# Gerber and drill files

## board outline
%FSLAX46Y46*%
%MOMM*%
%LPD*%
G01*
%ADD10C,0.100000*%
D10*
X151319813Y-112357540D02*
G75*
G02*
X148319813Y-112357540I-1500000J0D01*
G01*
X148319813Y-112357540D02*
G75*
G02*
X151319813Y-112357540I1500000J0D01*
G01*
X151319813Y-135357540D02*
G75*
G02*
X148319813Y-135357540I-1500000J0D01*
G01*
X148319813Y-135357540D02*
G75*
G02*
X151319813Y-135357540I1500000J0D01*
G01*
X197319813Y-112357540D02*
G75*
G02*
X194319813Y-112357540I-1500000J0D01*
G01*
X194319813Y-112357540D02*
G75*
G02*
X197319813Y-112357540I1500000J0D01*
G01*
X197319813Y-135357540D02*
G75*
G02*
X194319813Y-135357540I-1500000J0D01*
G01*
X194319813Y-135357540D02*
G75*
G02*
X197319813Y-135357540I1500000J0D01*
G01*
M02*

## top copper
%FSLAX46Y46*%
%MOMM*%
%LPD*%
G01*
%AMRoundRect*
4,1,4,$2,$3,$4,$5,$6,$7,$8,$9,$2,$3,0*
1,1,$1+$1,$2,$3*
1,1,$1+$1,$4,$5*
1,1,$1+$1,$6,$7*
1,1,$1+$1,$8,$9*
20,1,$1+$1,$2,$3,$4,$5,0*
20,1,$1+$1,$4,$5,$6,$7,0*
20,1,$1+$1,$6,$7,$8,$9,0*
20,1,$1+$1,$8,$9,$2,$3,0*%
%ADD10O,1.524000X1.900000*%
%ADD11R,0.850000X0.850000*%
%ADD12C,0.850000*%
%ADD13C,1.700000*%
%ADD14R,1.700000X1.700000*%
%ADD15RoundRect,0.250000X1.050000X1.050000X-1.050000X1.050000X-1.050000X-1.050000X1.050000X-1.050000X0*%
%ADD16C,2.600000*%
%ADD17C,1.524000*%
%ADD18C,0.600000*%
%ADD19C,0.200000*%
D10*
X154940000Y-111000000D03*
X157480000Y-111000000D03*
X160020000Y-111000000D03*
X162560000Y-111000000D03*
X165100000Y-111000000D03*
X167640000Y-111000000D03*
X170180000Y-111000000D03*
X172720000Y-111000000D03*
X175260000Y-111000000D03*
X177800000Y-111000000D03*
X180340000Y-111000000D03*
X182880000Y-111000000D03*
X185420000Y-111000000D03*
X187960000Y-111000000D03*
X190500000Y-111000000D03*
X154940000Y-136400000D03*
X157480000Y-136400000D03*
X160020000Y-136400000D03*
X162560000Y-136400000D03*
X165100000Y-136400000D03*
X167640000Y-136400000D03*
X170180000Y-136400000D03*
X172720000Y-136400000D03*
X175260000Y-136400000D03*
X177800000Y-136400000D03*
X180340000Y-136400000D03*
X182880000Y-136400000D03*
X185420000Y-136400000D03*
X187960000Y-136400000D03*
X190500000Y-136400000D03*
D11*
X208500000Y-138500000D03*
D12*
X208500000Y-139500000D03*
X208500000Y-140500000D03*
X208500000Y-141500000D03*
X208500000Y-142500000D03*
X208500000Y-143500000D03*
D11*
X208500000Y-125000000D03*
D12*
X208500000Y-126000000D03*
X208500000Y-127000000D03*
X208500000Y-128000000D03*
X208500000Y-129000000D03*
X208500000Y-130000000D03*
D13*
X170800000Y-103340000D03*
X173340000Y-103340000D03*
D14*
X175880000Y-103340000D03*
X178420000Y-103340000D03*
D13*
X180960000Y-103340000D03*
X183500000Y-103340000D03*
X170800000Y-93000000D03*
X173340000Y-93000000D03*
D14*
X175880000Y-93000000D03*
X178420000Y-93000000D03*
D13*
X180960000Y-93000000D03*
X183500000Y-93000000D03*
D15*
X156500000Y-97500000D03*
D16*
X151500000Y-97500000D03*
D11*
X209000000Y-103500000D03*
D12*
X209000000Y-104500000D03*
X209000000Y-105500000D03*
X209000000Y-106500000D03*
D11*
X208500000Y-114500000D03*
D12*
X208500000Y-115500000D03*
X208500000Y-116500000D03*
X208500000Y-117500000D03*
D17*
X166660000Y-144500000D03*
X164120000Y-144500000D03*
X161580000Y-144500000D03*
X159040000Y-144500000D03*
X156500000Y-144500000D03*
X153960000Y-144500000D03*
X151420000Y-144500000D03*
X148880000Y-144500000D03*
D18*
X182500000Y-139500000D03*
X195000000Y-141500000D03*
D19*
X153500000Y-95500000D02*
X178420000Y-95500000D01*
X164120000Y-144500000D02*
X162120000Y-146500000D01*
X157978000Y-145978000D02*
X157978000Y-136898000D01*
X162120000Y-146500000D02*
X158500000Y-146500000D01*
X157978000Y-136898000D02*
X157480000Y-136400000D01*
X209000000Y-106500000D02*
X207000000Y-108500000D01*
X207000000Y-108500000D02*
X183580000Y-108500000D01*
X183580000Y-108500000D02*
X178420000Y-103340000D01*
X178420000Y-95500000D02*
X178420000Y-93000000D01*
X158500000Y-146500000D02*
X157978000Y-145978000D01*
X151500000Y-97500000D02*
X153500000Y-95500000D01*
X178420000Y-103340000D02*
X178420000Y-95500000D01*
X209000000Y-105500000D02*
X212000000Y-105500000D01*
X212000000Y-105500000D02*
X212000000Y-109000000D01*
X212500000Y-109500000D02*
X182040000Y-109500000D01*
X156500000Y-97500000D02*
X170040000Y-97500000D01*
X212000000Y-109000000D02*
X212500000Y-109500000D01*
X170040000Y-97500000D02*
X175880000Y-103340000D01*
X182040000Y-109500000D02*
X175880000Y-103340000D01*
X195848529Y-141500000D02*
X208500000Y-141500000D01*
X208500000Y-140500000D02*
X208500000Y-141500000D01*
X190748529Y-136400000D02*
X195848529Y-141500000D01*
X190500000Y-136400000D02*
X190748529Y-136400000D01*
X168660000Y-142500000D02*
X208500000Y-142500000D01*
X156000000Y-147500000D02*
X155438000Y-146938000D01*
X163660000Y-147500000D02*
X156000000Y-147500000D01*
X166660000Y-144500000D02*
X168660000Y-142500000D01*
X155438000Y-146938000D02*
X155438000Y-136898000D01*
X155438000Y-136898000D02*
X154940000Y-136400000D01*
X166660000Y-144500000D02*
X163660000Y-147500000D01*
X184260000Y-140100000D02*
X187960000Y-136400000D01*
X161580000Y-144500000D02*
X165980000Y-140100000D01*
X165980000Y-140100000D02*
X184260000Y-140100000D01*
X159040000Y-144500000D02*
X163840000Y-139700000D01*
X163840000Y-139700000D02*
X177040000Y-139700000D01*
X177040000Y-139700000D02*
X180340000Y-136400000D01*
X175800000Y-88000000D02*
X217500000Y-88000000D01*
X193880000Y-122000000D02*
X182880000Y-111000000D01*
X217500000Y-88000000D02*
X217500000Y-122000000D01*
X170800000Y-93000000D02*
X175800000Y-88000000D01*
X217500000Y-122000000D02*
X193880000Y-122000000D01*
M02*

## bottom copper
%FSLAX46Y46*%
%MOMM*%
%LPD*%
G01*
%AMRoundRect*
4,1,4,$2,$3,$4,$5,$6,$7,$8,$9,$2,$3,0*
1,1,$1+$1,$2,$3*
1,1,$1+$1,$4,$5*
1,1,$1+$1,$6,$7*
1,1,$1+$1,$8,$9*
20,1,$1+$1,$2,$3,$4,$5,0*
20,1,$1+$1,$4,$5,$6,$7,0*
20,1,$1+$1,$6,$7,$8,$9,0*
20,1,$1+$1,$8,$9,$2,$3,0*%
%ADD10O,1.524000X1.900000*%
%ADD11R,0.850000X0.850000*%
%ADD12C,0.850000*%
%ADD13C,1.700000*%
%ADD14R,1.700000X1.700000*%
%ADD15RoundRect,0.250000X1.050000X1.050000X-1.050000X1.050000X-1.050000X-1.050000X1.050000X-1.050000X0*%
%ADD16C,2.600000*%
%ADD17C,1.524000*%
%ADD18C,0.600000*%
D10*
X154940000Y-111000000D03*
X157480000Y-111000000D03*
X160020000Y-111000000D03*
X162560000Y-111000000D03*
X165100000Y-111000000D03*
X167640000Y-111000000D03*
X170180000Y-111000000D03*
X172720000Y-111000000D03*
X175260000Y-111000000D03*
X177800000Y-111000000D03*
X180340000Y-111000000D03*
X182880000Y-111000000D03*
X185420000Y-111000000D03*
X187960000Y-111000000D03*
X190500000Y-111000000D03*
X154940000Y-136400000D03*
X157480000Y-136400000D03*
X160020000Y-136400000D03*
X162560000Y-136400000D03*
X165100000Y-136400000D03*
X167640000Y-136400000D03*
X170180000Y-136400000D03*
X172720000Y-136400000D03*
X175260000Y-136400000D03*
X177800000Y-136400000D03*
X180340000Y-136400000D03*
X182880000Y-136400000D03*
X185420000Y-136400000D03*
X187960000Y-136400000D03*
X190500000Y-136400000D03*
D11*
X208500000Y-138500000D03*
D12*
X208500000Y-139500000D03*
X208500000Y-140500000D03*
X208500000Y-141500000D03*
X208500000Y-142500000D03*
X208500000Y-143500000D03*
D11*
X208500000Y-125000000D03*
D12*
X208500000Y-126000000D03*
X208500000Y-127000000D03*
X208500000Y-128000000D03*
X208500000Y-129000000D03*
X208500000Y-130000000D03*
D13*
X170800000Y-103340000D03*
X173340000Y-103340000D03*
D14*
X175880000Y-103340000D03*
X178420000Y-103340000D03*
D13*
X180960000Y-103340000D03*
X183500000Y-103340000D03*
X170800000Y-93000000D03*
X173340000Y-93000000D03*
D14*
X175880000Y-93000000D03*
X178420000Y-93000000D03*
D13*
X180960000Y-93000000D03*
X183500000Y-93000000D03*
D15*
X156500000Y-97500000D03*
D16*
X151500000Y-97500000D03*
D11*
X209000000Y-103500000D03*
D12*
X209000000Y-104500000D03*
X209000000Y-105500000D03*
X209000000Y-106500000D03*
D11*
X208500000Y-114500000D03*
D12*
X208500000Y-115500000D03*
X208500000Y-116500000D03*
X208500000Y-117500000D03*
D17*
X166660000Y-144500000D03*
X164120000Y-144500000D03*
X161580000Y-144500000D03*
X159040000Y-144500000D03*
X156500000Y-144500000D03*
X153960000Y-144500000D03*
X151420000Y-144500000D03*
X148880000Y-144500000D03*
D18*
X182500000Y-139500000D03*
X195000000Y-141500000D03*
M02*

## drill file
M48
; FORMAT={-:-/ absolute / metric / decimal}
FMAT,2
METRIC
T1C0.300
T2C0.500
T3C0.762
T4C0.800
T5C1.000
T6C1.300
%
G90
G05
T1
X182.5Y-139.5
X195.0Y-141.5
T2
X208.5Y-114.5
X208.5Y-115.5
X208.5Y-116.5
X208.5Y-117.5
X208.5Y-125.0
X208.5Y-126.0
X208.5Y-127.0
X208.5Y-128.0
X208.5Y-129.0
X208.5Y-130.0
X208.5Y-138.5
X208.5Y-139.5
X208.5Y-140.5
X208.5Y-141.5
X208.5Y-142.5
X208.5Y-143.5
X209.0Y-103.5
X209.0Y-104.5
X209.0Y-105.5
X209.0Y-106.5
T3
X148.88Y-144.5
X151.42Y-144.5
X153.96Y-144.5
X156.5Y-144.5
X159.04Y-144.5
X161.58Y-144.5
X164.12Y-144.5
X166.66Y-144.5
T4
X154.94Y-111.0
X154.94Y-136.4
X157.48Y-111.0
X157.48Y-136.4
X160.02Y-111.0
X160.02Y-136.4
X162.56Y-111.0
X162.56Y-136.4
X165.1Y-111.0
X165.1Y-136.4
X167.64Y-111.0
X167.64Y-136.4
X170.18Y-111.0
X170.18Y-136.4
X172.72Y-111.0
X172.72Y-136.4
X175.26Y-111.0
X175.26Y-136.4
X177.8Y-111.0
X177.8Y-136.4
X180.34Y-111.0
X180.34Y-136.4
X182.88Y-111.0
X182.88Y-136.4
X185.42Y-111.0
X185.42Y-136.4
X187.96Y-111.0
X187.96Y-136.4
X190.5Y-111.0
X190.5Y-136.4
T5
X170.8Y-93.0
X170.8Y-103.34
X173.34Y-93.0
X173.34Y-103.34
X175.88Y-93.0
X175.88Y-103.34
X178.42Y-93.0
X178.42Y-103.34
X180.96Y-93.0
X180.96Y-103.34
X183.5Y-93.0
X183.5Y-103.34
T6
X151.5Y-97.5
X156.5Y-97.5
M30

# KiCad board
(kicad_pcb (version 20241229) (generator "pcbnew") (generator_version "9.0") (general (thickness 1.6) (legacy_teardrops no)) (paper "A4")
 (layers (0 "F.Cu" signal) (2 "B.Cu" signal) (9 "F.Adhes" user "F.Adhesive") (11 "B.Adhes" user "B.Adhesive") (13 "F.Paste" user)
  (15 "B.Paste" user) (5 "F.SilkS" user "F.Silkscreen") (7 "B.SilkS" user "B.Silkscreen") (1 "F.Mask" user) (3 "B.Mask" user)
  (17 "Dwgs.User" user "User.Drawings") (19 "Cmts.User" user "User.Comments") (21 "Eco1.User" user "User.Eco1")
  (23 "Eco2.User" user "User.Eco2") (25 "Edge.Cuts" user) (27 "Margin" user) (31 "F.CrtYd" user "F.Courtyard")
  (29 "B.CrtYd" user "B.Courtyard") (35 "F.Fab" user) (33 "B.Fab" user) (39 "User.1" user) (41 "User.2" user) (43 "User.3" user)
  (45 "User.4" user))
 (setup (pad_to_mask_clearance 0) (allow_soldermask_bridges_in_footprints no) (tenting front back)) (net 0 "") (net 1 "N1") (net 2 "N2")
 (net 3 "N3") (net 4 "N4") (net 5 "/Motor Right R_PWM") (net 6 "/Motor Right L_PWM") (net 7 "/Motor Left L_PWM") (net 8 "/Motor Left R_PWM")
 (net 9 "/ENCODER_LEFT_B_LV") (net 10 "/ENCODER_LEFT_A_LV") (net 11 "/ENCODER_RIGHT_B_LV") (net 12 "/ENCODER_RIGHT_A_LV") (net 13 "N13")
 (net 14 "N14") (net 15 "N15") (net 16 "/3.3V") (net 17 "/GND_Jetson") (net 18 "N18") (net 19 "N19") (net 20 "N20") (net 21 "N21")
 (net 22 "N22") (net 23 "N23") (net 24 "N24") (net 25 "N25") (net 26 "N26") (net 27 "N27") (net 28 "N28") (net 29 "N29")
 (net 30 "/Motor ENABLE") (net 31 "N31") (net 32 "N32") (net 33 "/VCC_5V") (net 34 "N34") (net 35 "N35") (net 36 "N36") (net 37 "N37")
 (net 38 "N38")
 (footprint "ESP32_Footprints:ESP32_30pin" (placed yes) (layer "F.Cu") (at 171.959813 122.92754 -90)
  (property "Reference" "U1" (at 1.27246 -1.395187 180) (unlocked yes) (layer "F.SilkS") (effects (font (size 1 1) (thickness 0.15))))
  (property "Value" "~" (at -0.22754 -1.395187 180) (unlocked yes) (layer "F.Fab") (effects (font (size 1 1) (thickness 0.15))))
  (fp_circle (center -10.57 22.14) (end -10.57 23.64) (stroke (width 0.1) (type default)) (fill no) (layer "Edge.Cuts"))
  (fp_circle (center 12.43 22.14) (end 12.43 23.64) (stroke (width 0.1) (type default)) (fill no) (layer "Edge.Cuts"))
  (fp_circle (center -10.57 -23.86) (end -10.57 -22.36) (stroke (width 0.1) (type default)) (fill no) (layer "Edge.Cuts"))
  (fp_circle (center 12.43 -23.86) (end 12.43 -22.36) (stroke (width 0.1) (type default)) (fill no) (layer "Edge.Cuts"))
  (pad "1" thru_hole oval (at -11.92754 17.019813 180) (size 1.524 1.9) (drill 0.8) (layers "*.Cu" "*.Mask") (remove_unused_layers no)
   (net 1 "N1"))
  (pad "2" thru_hole oval (at -11.92754 14.479813 180) (size 1.524 1.9) (drill 0.8) (layers "*.Cu" "*.Mask") (remove_unused_layers no)
   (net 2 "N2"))
  (pad "3" thru_hole oval (at -11.92754 11.939813 180) (size 1.524 1.9) (drill 0.8) (layers "*.Cu" "*.Mask") (remove_unused_layers no)
   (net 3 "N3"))
  (pad "4" thru_hole oval (at -11.92754 9.399813 180) (size 1.524 1.9) (drill 0.8) (layers "*.Cu" "*.Mask") (remove_unused_layers no)
   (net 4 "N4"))
  (pad "5" thru_hole oval (at -11.92754 6.859813 180) (size 1.524 1.9) (drill 0.8) (layers "*.Cu" "*.Mask") (remove_unused_layers no)
   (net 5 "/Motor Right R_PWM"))
  (pad "6" thru_hole oval (at -11.92754 4.319813 180) (size 1.524 1.9) (drill 0.8) (layers "*.Cu" "*.Mask") (remove_unused_layers no)
   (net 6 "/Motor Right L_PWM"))
  (pad "7" thru_hole oval (at -11.92754 1.779813 180) (size 1.524 1.9) (drill 0.8) (layers "*.Cu" "*.Mask") (remove_unused_layers no)
   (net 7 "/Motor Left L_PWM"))
  (pad "8" thru_hole oval (at -11.92754 -0.760187 180) (size 1.524 1.9) (drill 0.8) (layers "*.Cu" "*.Mask") (remove_unused_layers no)
   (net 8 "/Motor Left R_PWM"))
  (pad "9" thru_hole oval (at -11.92754 -3.300187 180) (size 1.524 1.9) (drill 0.8) (layers "*.Cu" "*.Mask") (remove_unused_layers no)
   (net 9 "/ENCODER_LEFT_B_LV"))
  (pad "10" thru_hole oval (at -11.92754 -5.840187 180) (size 1.524 1.9) (drill 0.8) (layers "*.Cu" "*.Mask") (remove_unused_layers no)
   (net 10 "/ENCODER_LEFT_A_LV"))
  (pad "11" thru_hole oval (at -11.92754 -8.380187 180) (size 1.524 1.9) (drill 0.8) (layers "*.Cu" "*.Mask") (remove_unused_layers no)
   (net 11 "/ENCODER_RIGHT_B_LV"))
  (pad "12" thru_hole oval (at -11.92754 -10.920187 180) (size 1.524 1.9) (drill 0.8) (layers "*.Cu" "*.Mask") (remove_unused_layers no)
   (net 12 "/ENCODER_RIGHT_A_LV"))
  (pad "13" thru_hole oval (at -11.92754 -13.460187 180) (size 1.524 1.9) (drill 0.8) (layers "*.Cu" "*.Mask") (remove_unused_layers no)
   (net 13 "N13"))
  (pad "14" thru_hole oval (at -11.92754 -16.000187 180) (size 1.524 1.9) (drill 0.8) (layers "*.Cu" "*.Mask") (remove_unused_layers no)
   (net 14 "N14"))
  (pad "15" thru_hole oval (at -11.92754 -18.540187 180) (size 1.524 1.9) (drill 0.8) (layers "*.Cu" "*.Mask") (remove_unused_layers no)
   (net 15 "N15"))
  (pad "16" thru_hole oval (at 13.47246 17.019813 180) (size 1.524 1.9) (drill 0.8) (layers "*.Cu" "*.Mask") (remove_unused_layers no)
   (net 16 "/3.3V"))
  (pad "17" thru_hole oval (at 13.47246 14.479813 180) (size 1.524 1.9) (drill 0.8) (layers "*.Cu" "*.Mask") (remove_unused_layers no)
   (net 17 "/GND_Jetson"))
  (pad "18" thru_hole oval (at 13.47246 11.939813 180) (size 1.524 1.9) (drill 0.8) (layers "*.Cu" "*.Mask") (remove_unused_layers no)
   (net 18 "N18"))
  (pad "19" thru_hole oval (at 13.47246 9.399813 180) (size 1.524 1.9) (drill 0.8) (layers "*.Cu" "*.Mask") (remove_unused_layers no)
   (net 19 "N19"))
  (pad "20" thru_hole oval (at 13.47246 6.859813 180) (size 1.524 1.9) (drill 0.8) (layers "*.Cu" "*.Mask" "Dwgs.User")
   (remove_unused_layers no) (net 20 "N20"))
  (pad "21" thru_hole oval (at 13.47246 4.319813 180) (size 1.524 1.9) (drill 0.8) (layers "*.Cu" "*.Mask") (remove_unused_layers no)
   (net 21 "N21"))
  (pad "22" thru_hole oval (at 13.47246 1.779813 180) (size 1.524 1.9) (drill 0.8) (layers "*.Cu" "*.Mask") (remove_unused_layers no)
   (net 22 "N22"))
  (pad "23" thru_hole oval (at 13.47246 -0.760187 180) (size 1.524 1.9) (drill 0.8) (layers "*.Cu" "*.Mask") (remove_unused_layers no)
   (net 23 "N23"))
  (pad "24" thru_hole oval (at 13.47246 -3.300187 180) (size 1.524 1.9) (drill 0.8) (layers "*.Cu" "*.Mask") (remove_unused_layers no)
   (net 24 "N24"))
  (pad "25" thru_hole oval (at 13.47246 -5.840187 180) (size 1.524 1.9) (drill 0.8) (layers "*.Cu" "*.Mask") (remove_unused_layers no)
   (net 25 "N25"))
  (pad "26" thru_hole oval (at 13.47246 -8.380187 180) (size 1.524 1.9) (drill 0.8) (layers "*.Cu" "*.Mask") (remove_unused_layers no)
   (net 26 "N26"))
  (pad "27" thru_hole oval (at 13.47246 -10.920187 180) (size 1.524 1.9) (drill 0.8) (layers "*.Cu" "*.Mask") (remove_unused_layers no)
   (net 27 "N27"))
  (pad "28" thru_hole oval (at 13.47246 -13.460187 180) (size 1.524 1.9) (drill 0.8) (layers "*.Cu" "*.Mask") (remove_unused_layers no)
   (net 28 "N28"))
  (pad "29" thru_hole oval (at 13.47246 -16.000187 180) (size 1.524 1.9) (drill 0.8) (layers "*.Cu" "*.Mask") (remove_unused_layers no)
   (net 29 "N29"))
  (pad "30" thru_hole oval (at 13.47246 -18.540187 180) (size 1.524 1.9) (drill 0.8) (layers "*.Cu" "*.Mask") (remove_unused_layers no)
   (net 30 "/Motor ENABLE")))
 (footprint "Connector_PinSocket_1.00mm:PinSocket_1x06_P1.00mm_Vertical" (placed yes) (layer "F.Cu") (at 208.5 138.5)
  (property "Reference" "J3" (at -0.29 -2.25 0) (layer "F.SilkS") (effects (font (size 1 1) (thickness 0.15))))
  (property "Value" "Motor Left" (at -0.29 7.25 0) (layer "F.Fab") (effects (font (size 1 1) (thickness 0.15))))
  (pad "1" thru_hole rect (at 0 0) (size 0.85 0.85) (drill 0.5) (layers "*.Cu" "*.Mask") (remove_unused_layers no)
   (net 8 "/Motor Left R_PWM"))
  (pad "2" thru_hole circle (at 0 1) (size 0.85 0.85) (drill 0.5) (layers "*.Cu" "*.Mask") (remove_unused_layers no)
   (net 7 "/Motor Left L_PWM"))
  (pad "3" thru_hole circle (at 0 2) (size 0.85 0.85) (drill 0.5) (layers "*.Cu" "*.Mask") (remove_unused_layers no)
   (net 30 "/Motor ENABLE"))
  (pad "4" thru_hole circle (at 0 3) (size 0.85 0.85) (drill 0.5) (layers "*.Cu" "*.Mask") (remove_unused_layers no)
   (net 30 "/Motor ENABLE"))
  (pad "5" thru_hole circle (at 0 4) (size 0.85 0.85) (drill 0.5) (layers "*.Cu" "*.Mask") (remove_unused_layers no) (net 16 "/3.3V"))
  (pad "6" thru_hole circle (at 0 5) (size 0.85 0.85) (drill 0.5) (layers "*.Cu" "*.Mask") (remove_unused_layers no) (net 17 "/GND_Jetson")))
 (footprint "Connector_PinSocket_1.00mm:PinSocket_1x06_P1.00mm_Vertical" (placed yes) (layer "F.Cu") (at 208.5 125)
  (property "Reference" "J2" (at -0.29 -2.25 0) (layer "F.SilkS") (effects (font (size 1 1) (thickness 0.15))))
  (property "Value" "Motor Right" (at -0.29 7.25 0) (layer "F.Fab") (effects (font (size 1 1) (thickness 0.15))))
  (pad "1" thru_hole rect (at 0 0) (size 0.85 0.85) (drill 0.5) (layers "*.Cu" "*.Mask") (remove_unused_layers no)
   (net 5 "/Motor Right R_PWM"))
  (pad "2" thru_hole circle (at 0 1) (size 0.85 0.85) (drill 0.5) (layers "*.Cu" "*.Mask") (remove_unused_layers no)
   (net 6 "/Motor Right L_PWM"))
  (pad "3" thru_hole circle (at 0 2) (size 0.85 0.85) (drill 0.5) (layers "*.Cu" "*.Mask") (remove_unused_layers no)
   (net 30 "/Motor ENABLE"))
  (pad "4" thru_hole circle (at 0 3) (size 0.85 0.85) (drill 0.5) (layers "*.Cu" "*.Mask") (remove_unused_layers no)
   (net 30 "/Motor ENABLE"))
  (pad "5" thru_hole circle (at 0 4) (size 0.85 0.85) (drill 0.5) (layers "*.Cu" "*.Mask") (remove_unused_layers no) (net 16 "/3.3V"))
  (pad "6" thru_hole circle (at 0 5) (size 0.85 0.85) (drill 0.5) (layers "*.Cu" "*.Mask") (remove_unused_layers no) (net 17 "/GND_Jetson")))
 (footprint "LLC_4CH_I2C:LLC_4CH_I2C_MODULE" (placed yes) (layer "F.Cu") (at 177.15 98.17 90)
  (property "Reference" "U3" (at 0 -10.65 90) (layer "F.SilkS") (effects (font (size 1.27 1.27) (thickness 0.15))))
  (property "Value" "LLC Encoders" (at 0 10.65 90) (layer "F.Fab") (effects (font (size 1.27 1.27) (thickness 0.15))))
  (pad "1" thru_hole circle (at -5.17 -6.35 90) (size 1.7 1.7) (drill 1) (layers "*.Cu" "*.Mask") (remove_unused_layers no) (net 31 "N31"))
  (pad "2" thru_hole circle (at -5.17 -3.81 90) (size 1.7 1.7) (drill 1) (layers "*.Cu" "*.Mask") (remove_unused_layers no) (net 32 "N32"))
  (pad "3" thru_hole rect (at -5.17 -1.27 90) (size 1.7 1.7) (drill 1) (layers "*.Cu" "*.Mask") (remove_unused_layers no) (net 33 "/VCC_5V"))
  (pad "4" thru_hole rect (at -5.17 1.27 90) (size 1.7 1.7) (drill 1) (layers "*.Cu" "*.Mask") (remove_unused_layers no)
   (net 17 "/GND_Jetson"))
  (pad "5" thru_hole circle (at -5.17 3.81 90) (size 1.7 1.7) (drill 1) (layers "*.Cu" "*.Mask") (remove_unused_layers no) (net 32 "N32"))
  (pad "6" thru_hole circle (at -5.17 6.35 90) (size 1.7 1.7) (drill 1) (layers "*.Cu" "*.Mask") (remove_unused_layers no) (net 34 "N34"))
  (pad "7" thru_hole circle (at 5.17 -6.35 90) (size 1.7 1.7) (drill 1) (layers "*.Cu" "*.Mask") (remove_unused_layers no)
   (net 12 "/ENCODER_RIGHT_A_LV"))
  (pad "8" thru_hole circle (at 5.17 -3.81 90) (size 1.7 1.7) (drill 1) (layers "*.Cu" "*.Mask") (remove_unused_layers no)
   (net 11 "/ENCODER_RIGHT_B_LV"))
  (pad "9" thru_hole rect (at 5.17 -1.27 90) (size 1.7 1.7) (drill 1) (layers "*.Cu" "*.Mask") (remove_unused_layers no) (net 16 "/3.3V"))
  (pad "10" thru_hole rect (at 5.17 1.27 90) (size 1.7 1.7) (drill 1) (layers "*.Cu" "*.Mask") (remove_unused_layers no)
   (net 17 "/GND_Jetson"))
  (pad "11" thru_hole circle (at 5.17 3.81 90) (size 1.7 1.7) (drill 1) (layers "*.Cu" "*.Mask") (remove_unused_layers no)
   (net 10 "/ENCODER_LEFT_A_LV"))
  (pad "12" thru_hole circle (at 5.17 6.35 90) (size 1.7 1.7) (drill 1) (layers "*.Cu" "*.Mask") (remove_unused_layers no)
   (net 9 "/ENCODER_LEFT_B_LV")))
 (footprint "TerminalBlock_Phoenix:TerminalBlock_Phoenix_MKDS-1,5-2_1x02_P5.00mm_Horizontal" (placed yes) (layer "F.Cu") (at 156.5 97.5 180)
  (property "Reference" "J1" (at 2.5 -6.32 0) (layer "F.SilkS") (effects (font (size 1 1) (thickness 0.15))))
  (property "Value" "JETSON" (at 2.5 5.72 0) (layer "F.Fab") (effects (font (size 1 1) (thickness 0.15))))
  (pad "1" thru_hole roundrect (at 0 0 180) (size 2.6 2.6) (drill 1.3) (layers "*.Cu" "*.Mask") (remove_unused_layers no)
   (roundrect_rratio 0.096154) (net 33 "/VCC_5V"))
  (pad "2" thru_hole circle (at 5 0 180) (size 2.6 2.6) (drill 1.3) (layers "*.Cu" "*.Mask") (remove_unused_layers no)
   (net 17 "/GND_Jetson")))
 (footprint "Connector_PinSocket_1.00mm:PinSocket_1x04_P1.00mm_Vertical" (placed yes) (layer "F.Cu") (at 209 103.5)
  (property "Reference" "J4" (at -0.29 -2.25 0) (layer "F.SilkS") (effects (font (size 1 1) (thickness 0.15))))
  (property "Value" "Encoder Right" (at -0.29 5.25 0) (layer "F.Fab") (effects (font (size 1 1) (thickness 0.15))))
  (pad "1" thru_hole rect (at 0 0) (size 0.85 0.85) (drill 0.5) (layers "*.Cu" "*.Mask") (remove_unused_layers no) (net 31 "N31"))
  (pad "2" thru_hole circle (at 0 1) (size 0.85 0.85) (drill 0.5) (layers "*.Cu" "*.Mask") (remove_unused_layers no) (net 32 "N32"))
  (pad "3" thru_hole circle (at 0 2) (size 0.85 0.85) (drill 0.5) (layers "*.Cu" "*.Mask") (remove_unused_layers no) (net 33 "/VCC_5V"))
  (pad "4" thru_hole circle (at 0 3) (size 0.85 0.85) (drill 0.5) (layers "*.Cu" "*.Mask") (remove_unused_layers no) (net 17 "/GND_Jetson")))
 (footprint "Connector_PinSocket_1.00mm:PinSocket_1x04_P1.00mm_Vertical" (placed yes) (layer "F.Cu") (at 208.5 114.5)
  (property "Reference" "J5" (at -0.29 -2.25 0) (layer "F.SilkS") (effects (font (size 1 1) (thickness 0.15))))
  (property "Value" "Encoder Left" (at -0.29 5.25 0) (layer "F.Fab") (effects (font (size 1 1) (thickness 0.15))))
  (pad "1" thru_hole rect (at 0 0) (size 0.85 0.85) (drill 0.5) (layers "*.Cu" "*.Mask") (remove_unused_layers no) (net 32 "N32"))
  (pad "2" thru_hole circle (at 0 1) (size 0.85 0.85) (drill 0.5) (layers "*.Cu" "*.Mask") (remove_unused_layers no) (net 34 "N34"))
  (pad "3" thru_hole circle (at 0 2) (size 0.85 0.85) (drill 0.5) (layers "*.Cu" "*.Mask") (remove_unused_layers no) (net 33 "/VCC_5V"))
  (pad "4" thru_hole circle (at 0 3) (size 0.85 0.85) (drill 0.5) (layers "*.Cu" "*.Mask") (remove_unused_layers no) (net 17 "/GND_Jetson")))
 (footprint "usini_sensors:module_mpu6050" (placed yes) (layer "F.Cu") (at 148.88 144.5 -90)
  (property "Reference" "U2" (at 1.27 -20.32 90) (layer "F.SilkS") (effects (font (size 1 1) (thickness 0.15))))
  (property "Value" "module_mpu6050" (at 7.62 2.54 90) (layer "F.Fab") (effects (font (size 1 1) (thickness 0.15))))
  (pad "1" thru_hole circle (at 0 -17.78 270) (size 1.524 1.524) (drill 0.762) (layers "*.Cu" "*.Mask") (remove_unused_layers no)
   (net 16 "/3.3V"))
  (pad "2" thru_hole circle (at 0 -15.24 270) (size 1.524 1.524) (drill 0.762) (layers "*.Cu" "*.Mask") (remove_unused_layers no)
   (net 17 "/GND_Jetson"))
  (pad "3" thru_hole circle (at 0 -12.7 270) (size 1.524 1.524) (drill 0.762) (layers "*.Cu" "*.Mask") (remove_unused_layers no)
   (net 29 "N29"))
  (pad "4" thru_hole circle (at 0 -10.16 270) (size 1.524 1.524) (drill 0.762) (layers "*.Cu" "*.Mask") (remove_unused_layers no)
   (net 26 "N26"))
  (pad "5" thru_hole circle (at 0 -7.62 270) (size 1.524 1.524) (drill 0.762) (layers "*.Cu" "*.Mask") (remove_unused_layers no)
   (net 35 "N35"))
  (pad "6" thru_hole circle (at 0 -5.08 270) (size 1.524 1.524) (drill 0.762) (layers "*.Cu" "*.Mask") (remove_unused_layers no)
   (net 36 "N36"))
  (pad "7" thru_hole circle (at 0 -2.54 270) (size 1.524 1.524) (drill 0.762) (layers "*.Cu" "*.Mask") (remove_unused_layers no)
   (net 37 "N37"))
  (pad "8" thru_hole circle (at 0 0 270) (size 1.524 1.524) (drill 0.762) (layers "*.Cu" "*.Mask") (remove_unused_layers no) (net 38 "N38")))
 (via (at 182.5 139.5) (size 0.6) (drill 0.3) (layers "F.Cu" "B.Cu") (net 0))
 (via (at 195 141.5) (size 0.6) (drill 0.3) (layers "F.Cu" "B.Cu") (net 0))
 (segment (start 153.5 95.5) (end 178.42 95.5) (width 0.2) (layer "F.Cu") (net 17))
 (segment (start 164.12 144.5) (end 162.12 146.5) (width 0.2) (layer "F.Cu") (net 17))
 (segment (start 157.978 145.978) (end 157.978 136.898) (width 0.2) (layer "F.Cu") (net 17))
 (segment (start 162.12 146.5) (end 158.5 146.5) (width 0.2) (layer "F.Cu") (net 17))
 (segment (start 157.978 136.898) (end 157.48 136.4) (width 0.2) (layer "F.Cu") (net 17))
 (segment (start 209 106.5) (end 207 108.5) (width 0.2) (layer "F.Cu") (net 17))
 (segment (start 207 108.5) (end 183.58 108.5) (width 0.2) (layer "F.Cu") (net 17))
 (segment (start 183.58 108.5) (end 178.42 103.34) (width 0.2) (layer "F.Cu") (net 17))
 (segment (start 178.42 95.5) (end 178.42 93) (width 0.2) (layer "F.Cu") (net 17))
 (segment (start 158.5 146.5) (end 157.978 145.978) (width 0.2) (layer "F.Cu") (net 17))
 (segment (start 151.5 97.5) (end 153.5 95.5) (width 0.2) (layer "F.Cu") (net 17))
 (segment (start 178.42 103.34) (end 178.42 95.5) (width 0.2) (layer "F.Cu") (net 17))
 (segment (start 209 105.5) (end 212 105.5) (width 0.2) (layer "F.Cu") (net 33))
 (segment (start 212 105.5) (end 212 109) (width 0.2) (layer "F.Cu") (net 33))
 (segment (start 212.5 109.5) (end 182.04 109.5) (width 0.2) (layer "F.Cu") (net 33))
 (segment (start 156.5 97.5) (end 170.04 97.5) (width 0.2) (layer "F.Cu") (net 33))
 (segment (start 212 109) (end 212.5 109.5) (width 0.2) (layer "F.Cu") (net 33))
 (segment (start 170.04 97.5) (end 175.88 103.34) (width 0.2) (layer "F.Cu") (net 33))
 (segment (start 182.04 109.5) (end 175.88 103.34) (width 0.2) (layer "F.Cu") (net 33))
 (segment (start 195.848529 141.5) (end 208.5 141.5) (width 0.2) (layer "F.Cu") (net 30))
 (segment (start 208.5 140.5) (end 208.5 141.5) (width 0.2) (layer "F.Cu") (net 30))
 (segment (start 190.748529 136.4) (end 195.848529 141.5) (width 0.2) (layer "F.Cu") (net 30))
 (segment (start 190.5 136.4) (end 190.748529 136.4) (width 0.2) (layer "F.Cu") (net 30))
 (segment (start 168.66 142.5) (end 208.5 142.5) (width 0.2) (layer "F.Cu") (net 16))
 (segment (start 156 147.5) (end 155.438 146.938) (width 0.2) (layer "F.Cu") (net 16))
 (segment (start 163.66 147.5) (end 156 147.5) (width 0.2) (layer "F.Cu") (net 16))
 (segment (start 166.66 144.5) (end 168.66 142.5) (width 0.2) (layer "F.Cu") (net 16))
 (segment (start 155.438 146.938) (end 155.438 136.898) (width 0.2) (layer "F.Cu") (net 16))
 (segment (start 155.438 136.898) (end 154.94 136.4) (width 0.2) (layer "F.Cu") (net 16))
 (segment (start 166.66 144.5) (end 163.66 147.5) (width 0.2) (layer "F.Cu") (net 16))
 (segment (start 184.26 140.1) (end 187.96 136.4) (width 0.2) (layer "F.Cu") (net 29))
 (segment (start 161.58 144.5) (end 165.98 140.1) (width 0.2) (layer "F.Cu") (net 29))
 (segment (start 165.98 140.1) (end 184.26 140.1) (width 0.2) (layer "F.Cu") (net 29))
 (segment (start 159.04 144.5) (end 163.84 139.7) (width 0.2) (layer "F.Cu") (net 26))
 (segment (start 163.84 139.7) (end 177.04 139.7) (width 0.2) (layer "F.Cu") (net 26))
 (segment (start 177.04 139.7) (end 180.34 136.4) (width 0.2) (layer "F.Cu") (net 26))
 (segment (start 175.8 88) (end 217.5 88) (width 0.2) (layer "F.Cu") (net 12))
 (segment (start 193.88 122) (end 182.88 111) (width 0.2) (layer "F.Cu") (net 12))
 (segment (start 217.5 88) (end 217.5 122) (width 0.2) (layer "F.Cu") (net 12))
 (segment (start 170.8 93) (end 175.8 88) (width 0.2) (layer "F.Cu") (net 12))
 (segment (start 217.5 122) (end 193.88 122) (width 0.2) (layer "F.Cu") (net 12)))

